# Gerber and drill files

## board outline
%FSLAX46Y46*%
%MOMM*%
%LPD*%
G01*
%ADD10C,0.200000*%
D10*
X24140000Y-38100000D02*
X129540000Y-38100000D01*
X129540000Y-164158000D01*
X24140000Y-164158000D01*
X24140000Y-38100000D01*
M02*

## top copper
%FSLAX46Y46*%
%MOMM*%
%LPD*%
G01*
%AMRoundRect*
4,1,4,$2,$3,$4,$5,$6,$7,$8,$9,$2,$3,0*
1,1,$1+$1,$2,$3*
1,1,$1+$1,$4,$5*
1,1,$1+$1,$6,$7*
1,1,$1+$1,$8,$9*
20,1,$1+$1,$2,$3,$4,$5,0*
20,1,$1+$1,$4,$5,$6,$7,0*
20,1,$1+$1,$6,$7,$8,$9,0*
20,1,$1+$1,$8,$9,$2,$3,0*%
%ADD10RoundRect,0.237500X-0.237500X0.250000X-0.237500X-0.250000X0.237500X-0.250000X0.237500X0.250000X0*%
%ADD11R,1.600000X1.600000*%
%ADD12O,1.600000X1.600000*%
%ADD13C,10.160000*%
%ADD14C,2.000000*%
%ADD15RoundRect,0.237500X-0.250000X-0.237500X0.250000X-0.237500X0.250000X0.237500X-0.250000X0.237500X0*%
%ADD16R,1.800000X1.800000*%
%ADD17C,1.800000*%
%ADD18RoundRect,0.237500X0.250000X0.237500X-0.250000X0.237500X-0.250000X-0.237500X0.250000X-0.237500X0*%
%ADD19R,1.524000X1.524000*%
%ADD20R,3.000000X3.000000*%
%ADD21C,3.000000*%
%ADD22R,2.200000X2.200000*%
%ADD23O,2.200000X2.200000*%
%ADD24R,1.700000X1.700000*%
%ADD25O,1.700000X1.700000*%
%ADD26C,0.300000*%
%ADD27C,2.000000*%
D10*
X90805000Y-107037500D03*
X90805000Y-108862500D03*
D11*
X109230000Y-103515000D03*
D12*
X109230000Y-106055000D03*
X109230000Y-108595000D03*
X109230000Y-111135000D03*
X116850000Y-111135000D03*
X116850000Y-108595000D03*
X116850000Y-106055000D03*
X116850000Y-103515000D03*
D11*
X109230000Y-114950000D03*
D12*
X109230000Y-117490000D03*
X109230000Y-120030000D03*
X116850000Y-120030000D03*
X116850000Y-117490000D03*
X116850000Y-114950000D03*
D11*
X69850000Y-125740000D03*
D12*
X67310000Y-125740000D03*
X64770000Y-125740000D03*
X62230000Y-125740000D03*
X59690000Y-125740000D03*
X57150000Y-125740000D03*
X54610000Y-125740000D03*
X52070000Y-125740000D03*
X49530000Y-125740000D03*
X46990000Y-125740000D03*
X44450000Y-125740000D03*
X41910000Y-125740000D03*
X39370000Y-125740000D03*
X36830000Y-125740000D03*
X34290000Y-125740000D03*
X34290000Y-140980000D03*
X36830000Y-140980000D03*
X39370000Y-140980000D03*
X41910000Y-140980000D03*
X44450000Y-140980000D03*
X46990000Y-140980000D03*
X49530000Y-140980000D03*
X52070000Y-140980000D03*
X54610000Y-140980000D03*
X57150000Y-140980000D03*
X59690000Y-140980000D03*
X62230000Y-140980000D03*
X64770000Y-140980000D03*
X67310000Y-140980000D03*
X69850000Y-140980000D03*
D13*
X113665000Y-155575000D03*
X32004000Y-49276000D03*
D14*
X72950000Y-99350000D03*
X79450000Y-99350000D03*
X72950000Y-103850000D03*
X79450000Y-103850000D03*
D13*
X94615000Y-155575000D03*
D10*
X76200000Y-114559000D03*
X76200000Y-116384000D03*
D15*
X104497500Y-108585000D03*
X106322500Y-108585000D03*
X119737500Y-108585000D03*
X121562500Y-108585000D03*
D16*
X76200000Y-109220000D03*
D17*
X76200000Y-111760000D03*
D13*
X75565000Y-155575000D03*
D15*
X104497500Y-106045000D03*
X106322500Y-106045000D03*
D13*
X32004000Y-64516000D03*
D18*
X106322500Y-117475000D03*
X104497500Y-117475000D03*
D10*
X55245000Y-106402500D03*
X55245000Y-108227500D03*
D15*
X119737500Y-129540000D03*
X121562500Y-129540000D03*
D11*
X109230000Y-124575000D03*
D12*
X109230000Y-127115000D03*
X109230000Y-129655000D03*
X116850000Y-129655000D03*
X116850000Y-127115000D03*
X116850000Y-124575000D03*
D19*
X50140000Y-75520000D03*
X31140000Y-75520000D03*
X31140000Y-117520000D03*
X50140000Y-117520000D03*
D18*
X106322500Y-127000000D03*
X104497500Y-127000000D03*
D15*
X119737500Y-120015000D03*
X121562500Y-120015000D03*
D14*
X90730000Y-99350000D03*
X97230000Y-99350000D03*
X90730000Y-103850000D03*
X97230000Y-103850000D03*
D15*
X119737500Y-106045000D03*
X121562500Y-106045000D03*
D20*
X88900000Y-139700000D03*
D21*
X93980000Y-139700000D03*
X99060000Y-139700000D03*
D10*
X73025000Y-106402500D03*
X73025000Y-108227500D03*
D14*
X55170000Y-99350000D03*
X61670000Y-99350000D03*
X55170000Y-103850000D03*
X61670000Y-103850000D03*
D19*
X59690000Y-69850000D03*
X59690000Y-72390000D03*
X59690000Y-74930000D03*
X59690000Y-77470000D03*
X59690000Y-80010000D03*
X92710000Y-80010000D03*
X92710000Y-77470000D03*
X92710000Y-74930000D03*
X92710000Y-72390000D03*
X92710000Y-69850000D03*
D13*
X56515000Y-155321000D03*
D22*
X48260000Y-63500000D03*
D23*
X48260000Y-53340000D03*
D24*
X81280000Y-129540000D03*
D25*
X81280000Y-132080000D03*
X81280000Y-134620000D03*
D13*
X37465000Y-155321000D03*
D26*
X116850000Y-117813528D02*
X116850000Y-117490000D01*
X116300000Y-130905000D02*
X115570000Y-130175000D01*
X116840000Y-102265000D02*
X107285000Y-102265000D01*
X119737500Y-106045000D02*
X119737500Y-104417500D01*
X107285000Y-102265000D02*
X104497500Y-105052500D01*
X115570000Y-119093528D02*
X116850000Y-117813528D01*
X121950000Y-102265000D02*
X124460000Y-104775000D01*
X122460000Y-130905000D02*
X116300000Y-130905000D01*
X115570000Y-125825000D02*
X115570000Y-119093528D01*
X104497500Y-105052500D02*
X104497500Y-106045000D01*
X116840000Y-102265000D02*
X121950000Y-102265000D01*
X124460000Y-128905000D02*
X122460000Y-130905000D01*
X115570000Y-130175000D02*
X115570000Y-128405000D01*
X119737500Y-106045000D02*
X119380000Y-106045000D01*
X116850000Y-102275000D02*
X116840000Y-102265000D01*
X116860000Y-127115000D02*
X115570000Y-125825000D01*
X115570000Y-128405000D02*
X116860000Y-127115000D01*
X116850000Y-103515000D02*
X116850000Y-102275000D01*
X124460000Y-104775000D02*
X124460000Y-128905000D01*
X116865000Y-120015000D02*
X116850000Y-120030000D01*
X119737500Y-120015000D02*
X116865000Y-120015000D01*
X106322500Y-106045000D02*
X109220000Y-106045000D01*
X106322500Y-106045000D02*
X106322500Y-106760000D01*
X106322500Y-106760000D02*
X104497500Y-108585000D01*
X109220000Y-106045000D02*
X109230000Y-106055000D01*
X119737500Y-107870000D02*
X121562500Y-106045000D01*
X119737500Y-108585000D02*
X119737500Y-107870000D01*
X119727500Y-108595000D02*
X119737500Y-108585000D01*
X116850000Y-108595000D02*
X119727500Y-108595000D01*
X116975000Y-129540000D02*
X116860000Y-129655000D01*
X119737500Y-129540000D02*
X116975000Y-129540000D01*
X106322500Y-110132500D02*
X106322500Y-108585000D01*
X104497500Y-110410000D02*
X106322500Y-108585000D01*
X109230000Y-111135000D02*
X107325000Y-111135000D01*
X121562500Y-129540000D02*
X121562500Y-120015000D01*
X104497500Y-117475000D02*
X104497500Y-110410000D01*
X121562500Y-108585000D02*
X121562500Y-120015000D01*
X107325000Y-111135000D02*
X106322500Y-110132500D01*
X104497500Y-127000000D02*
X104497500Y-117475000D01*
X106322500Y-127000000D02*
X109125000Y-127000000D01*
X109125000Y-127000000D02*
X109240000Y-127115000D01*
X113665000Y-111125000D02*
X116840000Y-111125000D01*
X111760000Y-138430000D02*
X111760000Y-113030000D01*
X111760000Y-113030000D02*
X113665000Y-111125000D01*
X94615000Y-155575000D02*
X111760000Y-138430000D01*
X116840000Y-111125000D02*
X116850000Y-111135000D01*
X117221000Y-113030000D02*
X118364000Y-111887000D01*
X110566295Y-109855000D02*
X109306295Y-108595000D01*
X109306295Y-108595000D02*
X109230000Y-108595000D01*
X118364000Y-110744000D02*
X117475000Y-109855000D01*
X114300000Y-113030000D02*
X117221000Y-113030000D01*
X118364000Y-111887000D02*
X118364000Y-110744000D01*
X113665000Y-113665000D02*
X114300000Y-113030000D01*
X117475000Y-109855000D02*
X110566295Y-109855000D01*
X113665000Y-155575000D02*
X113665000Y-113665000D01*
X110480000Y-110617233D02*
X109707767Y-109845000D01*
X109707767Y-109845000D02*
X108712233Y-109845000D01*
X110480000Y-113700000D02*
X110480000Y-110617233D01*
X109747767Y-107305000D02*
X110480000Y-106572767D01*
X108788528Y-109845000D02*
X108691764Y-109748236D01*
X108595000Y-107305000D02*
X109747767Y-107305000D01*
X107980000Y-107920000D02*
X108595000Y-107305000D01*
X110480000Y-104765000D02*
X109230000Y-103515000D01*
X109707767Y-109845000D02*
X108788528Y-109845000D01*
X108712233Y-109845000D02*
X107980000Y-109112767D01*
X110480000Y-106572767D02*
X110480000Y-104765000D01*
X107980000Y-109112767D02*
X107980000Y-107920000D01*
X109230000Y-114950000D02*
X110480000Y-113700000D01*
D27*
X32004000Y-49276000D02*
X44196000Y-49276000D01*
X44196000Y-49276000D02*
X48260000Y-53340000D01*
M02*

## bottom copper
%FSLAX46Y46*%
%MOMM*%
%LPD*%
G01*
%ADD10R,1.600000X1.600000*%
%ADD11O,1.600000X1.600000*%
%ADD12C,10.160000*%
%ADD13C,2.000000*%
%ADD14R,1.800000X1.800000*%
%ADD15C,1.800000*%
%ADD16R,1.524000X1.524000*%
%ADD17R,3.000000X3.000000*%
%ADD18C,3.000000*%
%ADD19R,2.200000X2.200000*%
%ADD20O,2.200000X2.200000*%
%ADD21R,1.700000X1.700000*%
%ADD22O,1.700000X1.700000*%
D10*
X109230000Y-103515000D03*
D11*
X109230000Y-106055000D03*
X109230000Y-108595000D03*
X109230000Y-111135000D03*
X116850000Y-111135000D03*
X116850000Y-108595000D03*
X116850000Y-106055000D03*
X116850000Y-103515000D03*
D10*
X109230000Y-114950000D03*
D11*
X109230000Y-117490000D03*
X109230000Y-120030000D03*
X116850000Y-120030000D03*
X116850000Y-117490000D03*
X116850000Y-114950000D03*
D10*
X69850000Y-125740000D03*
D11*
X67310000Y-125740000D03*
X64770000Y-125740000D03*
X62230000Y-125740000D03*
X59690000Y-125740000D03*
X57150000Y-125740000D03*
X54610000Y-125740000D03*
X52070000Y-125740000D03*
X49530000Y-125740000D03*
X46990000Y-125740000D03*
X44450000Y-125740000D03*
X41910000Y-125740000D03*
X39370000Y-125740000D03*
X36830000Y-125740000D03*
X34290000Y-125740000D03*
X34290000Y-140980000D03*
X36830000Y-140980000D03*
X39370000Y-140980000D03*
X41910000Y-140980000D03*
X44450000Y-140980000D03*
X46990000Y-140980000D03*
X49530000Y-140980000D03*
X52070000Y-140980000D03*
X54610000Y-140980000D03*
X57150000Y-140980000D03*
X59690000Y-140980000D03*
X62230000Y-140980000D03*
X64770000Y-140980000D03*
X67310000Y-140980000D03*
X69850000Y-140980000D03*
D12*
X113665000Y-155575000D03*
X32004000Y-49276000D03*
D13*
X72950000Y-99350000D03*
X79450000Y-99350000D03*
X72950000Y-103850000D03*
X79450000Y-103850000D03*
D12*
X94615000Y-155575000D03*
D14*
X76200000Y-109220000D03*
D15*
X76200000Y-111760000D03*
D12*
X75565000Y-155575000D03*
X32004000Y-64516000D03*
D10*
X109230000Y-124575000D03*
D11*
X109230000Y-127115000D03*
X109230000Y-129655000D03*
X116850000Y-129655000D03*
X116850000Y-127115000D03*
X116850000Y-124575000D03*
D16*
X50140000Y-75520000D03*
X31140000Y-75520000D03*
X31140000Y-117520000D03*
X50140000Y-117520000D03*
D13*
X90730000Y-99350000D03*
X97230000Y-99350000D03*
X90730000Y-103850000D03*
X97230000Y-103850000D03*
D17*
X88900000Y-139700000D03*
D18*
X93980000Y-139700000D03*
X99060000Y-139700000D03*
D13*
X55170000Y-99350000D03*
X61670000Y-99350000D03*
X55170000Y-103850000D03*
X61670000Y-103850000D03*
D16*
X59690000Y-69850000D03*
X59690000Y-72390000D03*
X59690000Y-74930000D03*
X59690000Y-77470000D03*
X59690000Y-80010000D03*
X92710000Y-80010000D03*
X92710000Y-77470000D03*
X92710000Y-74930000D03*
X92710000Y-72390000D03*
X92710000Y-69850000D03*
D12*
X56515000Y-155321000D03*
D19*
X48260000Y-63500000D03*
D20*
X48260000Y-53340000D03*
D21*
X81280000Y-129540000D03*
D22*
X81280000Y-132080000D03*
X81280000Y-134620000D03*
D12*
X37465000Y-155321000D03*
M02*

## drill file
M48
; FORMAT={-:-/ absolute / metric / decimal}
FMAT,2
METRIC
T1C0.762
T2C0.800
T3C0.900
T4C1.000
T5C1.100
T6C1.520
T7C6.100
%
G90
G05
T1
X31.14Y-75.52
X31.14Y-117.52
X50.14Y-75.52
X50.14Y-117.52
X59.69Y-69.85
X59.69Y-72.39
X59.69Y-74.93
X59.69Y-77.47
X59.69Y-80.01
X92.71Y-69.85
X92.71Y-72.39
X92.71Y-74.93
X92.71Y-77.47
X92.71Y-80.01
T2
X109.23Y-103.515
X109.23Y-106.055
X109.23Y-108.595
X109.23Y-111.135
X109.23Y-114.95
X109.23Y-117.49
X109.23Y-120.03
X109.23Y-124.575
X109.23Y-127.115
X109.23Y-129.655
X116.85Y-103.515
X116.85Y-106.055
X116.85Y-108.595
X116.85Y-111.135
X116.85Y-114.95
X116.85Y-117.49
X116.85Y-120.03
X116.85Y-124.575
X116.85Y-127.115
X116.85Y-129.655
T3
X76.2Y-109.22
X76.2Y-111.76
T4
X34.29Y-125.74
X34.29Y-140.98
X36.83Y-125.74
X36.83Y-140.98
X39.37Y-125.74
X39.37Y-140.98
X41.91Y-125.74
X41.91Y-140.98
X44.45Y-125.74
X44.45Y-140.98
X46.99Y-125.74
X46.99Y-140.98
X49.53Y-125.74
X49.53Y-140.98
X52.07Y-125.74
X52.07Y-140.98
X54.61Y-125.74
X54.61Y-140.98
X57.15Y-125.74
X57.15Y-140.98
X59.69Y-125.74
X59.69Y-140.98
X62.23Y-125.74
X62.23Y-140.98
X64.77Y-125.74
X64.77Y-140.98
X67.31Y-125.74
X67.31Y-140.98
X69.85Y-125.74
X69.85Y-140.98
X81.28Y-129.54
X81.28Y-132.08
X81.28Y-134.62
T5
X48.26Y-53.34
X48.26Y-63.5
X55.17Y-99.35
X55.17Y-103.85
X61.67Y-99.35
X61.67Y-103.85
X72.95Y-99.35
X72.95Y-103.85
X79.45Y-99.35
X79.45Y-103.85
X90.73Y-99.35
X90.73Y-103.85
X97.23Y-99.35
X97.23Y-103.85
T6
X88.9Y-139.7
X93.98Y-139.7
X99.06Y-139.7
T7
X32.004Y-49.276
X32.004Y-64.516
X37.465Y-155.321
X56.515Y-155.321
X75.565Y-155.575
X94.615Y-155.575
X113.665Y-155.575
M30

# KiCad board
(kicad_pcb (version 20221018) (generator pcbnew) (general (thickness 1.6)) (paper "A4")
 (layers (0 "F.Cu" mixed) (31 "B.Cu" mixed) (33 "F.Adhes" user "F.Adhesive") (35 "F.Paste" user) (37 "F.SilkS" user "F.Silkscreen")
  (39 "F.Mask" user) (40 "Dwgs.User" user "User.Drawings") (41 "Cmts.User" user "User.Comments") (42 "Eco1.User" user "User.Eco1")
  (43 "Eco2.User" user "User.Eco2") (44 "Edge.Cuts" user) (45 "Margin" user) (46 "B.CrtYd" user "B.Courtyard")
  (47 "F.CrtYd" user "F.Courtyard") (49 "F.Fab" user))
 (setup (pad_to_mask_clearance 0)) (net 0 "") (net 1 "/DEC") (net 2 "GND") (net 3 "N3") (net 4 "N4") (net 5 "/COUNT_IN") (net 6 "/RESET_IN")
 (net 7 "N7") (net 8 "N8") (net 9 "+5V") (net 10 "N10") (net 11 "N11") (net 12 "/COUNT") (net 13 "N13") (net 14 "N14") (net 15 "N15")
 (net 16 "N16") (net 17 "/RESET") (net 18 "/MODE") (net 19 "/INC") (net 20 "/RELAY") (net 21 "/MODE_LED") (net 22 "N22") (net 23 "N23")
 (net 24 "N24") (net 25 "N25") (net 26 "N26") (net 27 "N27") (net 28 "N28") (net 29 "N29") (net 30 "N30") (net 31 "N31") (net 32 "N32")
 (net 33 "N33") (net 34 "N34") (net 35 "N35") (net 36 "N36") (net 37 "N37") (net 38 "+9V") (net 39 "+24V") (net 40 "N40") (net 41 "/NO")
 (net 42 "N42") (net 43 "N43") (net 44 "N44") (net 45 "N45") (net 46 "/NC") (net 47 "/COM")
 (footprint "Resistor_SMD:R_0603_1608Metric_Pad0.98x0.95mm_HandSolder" (layer "F.Cu") (at 90.805 107.95 -90)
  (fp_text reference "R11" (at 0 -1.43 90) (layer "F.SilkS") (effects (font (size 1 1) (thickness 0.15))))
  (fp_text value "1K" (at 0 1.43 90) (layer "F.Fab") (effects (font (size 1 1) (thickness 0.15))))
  (pad "1" smd roundrect (at -0.9125 0 270) (size 0.975 0.95) (layers "F.Cu" "F.Paste" "F.Mask") (roundrect_rratio 0.25) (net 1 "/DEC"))
  (pad "2" smd roundrect (at 0.9125 0 270) (size 0.975 0.95) (layers "F.Cu" "F.Paste" "F.Mask") (roundrect_rratio 0.25) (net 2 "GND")))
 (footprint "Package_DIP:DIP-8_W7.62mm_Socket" (layer "F.Cu") (at 109.23 103.515)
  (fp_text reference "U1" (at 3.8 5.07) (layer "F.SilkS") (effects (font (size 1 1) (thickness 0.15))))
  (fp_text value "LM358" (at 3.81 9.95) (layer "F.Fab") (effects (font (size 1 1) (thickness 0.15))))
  (pad "1" thru_hole rect (at 0 0) (size 1.6 1.6) (drill 0.8) (layers "*.Cu" "*.Mask") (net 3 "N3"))
  (pad "2" thru_hole oval (at 0 2.54) (size 1.6 1.6) (drill 0.8) (layers "*.Cu" "*.Mask") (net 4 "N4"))
  (pad "3" thru_hole oval (at 0 5.08) (size 1.6 1.6) (drill 0.8) (layers "*.Cu" "*.Mask") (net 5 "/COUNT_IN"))
  (pad "4" thru_hole oval (at 0 7.62) (size 1.6 1.6) (drill 0.8) (layers "*.Cu" "*.Mask") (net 2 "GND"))
  (pad "5" thru_hole oval (at 7.62 7.62) (size 1.6 1.6) (drill 0.8) (layers "*.Cu" "*.Mask") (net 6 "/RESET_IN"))
  (pad "6" thru_hole oval (at 7.62 5.08) (size 1.6 1.6) (drill 0.8) (layers "*.Cu" "*.Mask") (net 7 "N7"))
  (pad "7" thru_hole oval (at 7.62 2.54) (size 1.6 1.6) (drill 0.8) (layers "*.Cu" "*.Mask") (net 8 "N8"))
  (pad "8" thru_hole oval (at 7.62 0) (size 1.6 1.6) (drill 0.8) (layers "*.Cu" "*.Mask") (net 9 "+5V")))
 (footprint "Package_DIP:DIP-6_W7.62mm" (layer "F.Cu") (at 109.23 114.95)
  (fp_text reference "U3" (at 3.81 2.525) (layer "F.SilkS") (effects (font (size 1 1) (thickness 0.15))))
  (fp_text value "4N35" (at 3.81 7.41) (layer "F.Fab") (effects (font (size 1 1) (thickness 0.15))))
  (pad "1" thru_hole rect (at 0 0) (size 1.6 1.6) (drill 0.8) (layers "*.Cu" "*.Mask") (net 3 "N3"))
  (pad "2" thru_hole oval (at 0 2.54) (size 1.6 1.6) (drill 0.8) (layers "*.Cu" "*.Mask") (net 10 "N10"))
  (pad "3" thru_hole oval (at 0 5.08) (size 1.6 1.6) (drill 0.8) (layers "*.Cu" "*.Mask") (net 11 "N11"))
  (pad "4" thru_hole oval (at 7.62 5.08) (size 1.6 1.6) (drill 0.8) (layers "*.Cu" "*.Mask") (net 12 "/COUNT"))
  (pad "5" thru_hole oval (at 7.62 2.54) (size 1.6 1.6) (drill 0.8) (layers "*.Cu" "*.Mask") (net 9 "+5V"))
  (pad "6" thru_hole oval (at 7.62 0) (size 1.6 1.6) (drill 0.8) (layers "*.Cu" "*.Mask") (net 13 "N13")))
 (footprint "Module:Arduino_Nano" (layer "F.Cu") (at 69.85 125.74 -90)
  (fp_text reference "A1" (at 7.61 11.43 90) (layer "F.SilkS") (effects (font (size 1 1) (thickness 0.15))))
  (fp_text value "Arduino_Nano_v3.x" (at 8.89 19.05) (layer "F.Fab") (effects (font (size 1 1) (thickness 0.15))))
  (pad "1" thru_hole rect (at 0 0 270) (size 1.6 1.6) (drill 1) (layers "*.Cu" "*.Mask") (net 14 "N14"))
  (pad "2" thru_hole oval (at 0 2.54 270) (size 1.6 1.6) (drill 1) (layers "*.Cu" "*.Mask") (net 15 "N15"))
  (pad "3" thru_hole oval (at 0 5.08 270) (size 1.6 1.6) (drill 1) (layers "*.Cu" "*.Mask") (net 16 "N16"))
  (pad "4" thru_hole oval (at 0 7.62 270) (size 1.6 1.6) (drill 1) (layers "*.Cu" "*.Mask") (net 2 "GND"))
  (pad "5" thru_hole oval (at 0 10.16 270) (size 1.6 1.6) (drill 1) (layers "*.Cu" "*.Mask") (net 12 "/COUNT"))
  (pad "6" thru_hole oval (at 0 12.7 270) (size 1.6 1.6) (drill 1) (layers "*.Cu" "*.Mask") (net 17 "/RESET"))
  (pad "7" thru_hole oval (at 0 15.24 270) (size 1.6 1.6) (drill 1) (layers "*.Cu" "*.Mask") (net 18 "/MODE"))
  (pad "8" thru_hole oval (at 0 17.78 270) (size 1.6 1.6) (drill 1) (layers "*.Cu" "*.Mask") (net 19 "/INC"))
  (pad "9" thru_hole oval (at 0 20.32 270) (size 1.6 1.6) (drill 1) (layers "*.Cu" "*.Mask") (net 1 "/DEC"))
  (pad "10" thru_hole oval (at 0 22.86 270) (size 1.6 1.6) (drill 1) (layers "*.Cu" "*.Mask") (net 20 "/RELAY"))
  (pad "11" thru_hole oval (at 0 25.4 270) (size 1.6 1.6) (drill 1) (layers "*.Cu" "*.Mask") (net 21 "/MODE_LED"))
  (pad "12" thru_hole oval (at 0 27.94 270) (size 1.6 1.6) (drill 1) (layers "*.Cu" "*.Mask") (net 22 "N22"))
  (pad "13" thru_hole oval (at 0 30.48 270) (size 1.6 1.6) (drill 1) (layers "*.Cu" "*.Mask") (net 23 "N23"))
  (pad "14" thru_hole oval (at 0 33.02 270) (size 1.6 1.6) (drill 1) (layers "*.Cu" "*.Mask") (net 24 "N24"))
  (pad "15" thru_hole oval (at 0 35.56 270) (size 1.6 1.6) (drill 1) (layers "*.Cu" "*.Mask") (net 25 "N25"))
  (pad "16" thru_hole oval (at 15.24 35.56 270) (size 1.6 1.6) (drill 1) (layers "*.Cu" "*.Mask") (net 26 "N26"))
  (pad "17" thru_hole oval (at 15.24 33.02 270) (size 1.6 1.6) (drill 1) (layers "*.Cu" "*.Mask") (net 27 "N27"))
  (pad "18" thru_hole oval (at 15.24 30.48 270) (size 1.6 1.6) (drill 1) (layers "*.Cu" "*.Mask") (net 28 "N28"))
  (pad "19" thru_hole oval (at 15.24 27.94 270) (size 1.6 1.6) (drill 1) (layers "*.Cu" "*.Mask") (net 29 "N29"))
  (pad "20" thru_hole oval (at 15.24 25.4 270) (size 1.6 1.6) (drill 1) (layers "*.Cu" "*.Mask") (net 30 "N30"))
  (pad "21" thru_hole oval (at 15.24 22.86 270) (size 1.6 1.6) (drill 1) (layers "*.Cu" "*.Mask") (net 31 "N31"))
  (pad "22" thru_hole oval (at 15.24 20.32 270) (size 1.6 1.6) (drill 1) (layers "*.Cu" "*.Mask") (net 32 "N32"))
  (pad "23" thru_hole oval (at 15.24 17.78 270) (size 1.6 1.6) (drill 1) (layers "*.Cu" "*.Mask") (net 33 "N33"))
  (pad "24" thru_hole oval (at 15.24 15.24 270) (size 1.6 1.6) (drill 1) (layers "*.Cu" "*.Mask") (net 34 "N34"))
  (pad "25" thru_hole oval (at 15.24 12.7 270) (size 1.6 1.6) (drill 1) (layers "*.Cu" "*.Mask") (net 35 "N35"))
  (pad "26" thru_hole oval (at 15.24 10.16 270) (size 1.6 1.6) (drill 1) (layers "*.Cu" "*.Mask") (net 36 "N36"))
  (pad "27" thru_hole oval (at 15.24 7.62 270) (size 1.6 1.6) (drill 1) (layers "*.Cu" "*.Mask") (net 9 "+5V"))
  (pad "28" thru_hole oval (at 15.24 5.08 270) (size 1.6 1.6) (drill 1) (layers "*.Cu" "*.Mask") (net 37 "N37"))
  (pad "29" thru_hole oval (at 15.24 2.54 270) (size 1.6 1.6) (drill 1) (layers "*.Cu" "*.Mask") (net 2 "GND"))
  (pad "30" thru_hole oval (at 15.24 0 270) (size 1.6 1.6) (drill 1) (layers "*.Cu" "*.Mask") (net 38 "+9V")))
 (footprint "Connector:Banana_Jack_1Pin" (layer "F.Cu") (at 113.665 155.575)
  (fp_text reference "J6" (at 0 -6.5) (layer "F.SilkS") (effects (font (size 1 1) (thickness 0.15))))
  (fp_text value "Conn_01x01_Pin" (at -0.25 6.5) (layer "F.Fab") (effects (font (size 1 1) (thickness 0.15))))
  (pad "1" thru_hole circle (at 0 0) (size 10.16 10.16) (drill 6.1) (layers "*.Cu" "*.Mask") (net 5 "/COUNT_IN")))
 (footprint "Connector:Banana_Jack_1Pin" (layer "F.Cu") (at 32.004 49.276)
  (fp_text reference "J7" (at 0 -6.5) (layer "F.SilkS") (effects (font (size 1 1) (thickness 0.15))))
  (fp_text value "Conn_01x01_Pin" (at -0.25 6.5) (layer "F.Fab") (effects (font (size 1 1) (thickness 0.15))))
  (pad "1" thru_hole circle (at 0 0) (size 10.16 10.16) (drill 6.1) (layers "*.Cu" "*.Mask") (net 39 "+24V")))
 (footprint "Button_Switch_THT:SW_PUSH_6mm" (layer "F.Cu") (at 72.95 99.35)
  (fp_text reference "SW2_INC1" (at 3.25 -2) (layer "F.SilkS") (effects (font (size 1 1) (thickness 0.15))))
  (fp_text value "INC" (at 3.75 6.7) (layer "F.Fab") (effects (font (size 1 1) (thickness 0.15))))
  (pad "1" thru_hole circle (at 0 0 90) (size 2 2) (drill 1.1) (layers "*.Cu" "*.Mask") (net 9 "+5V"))
  (pad "1" thru_hole circle (at 6.5 0 90) (size 2 2) (drill 1.1) (layers "*.Cu" "*.Mask") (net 9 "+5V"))
  (pad "2" thru_hole circle (at 0 4.5 90) (size 2 2) (drill 1.1) (layers "*.Cu" "*.Mask") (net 19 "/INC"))
  (pad "2" thru_hole circle (at 6.5 4.5 90) (size 2 2) (drill 1.1) (layers "*.Cu" "*.Mask") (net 19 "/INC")))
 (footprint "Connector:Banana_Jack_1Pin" (layer "F.Cu") (at 94.615 155.575)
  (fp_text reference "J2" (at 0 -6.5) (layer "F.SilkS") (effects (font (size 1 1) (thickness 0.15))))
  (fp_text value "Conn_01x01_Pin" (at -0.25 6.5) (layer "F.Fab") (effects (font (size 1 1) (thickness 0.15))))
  (pad "1" thru_hole circle (at 0 0) (size 10.16 10.16) (drill 6.1) (layers "*.Cu" "*.Mask") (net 6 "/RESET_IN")))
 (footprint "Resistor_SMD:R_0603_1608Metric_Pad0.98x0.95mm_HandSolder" (layer "F.Cu") (at 76.2 115.4715 -90)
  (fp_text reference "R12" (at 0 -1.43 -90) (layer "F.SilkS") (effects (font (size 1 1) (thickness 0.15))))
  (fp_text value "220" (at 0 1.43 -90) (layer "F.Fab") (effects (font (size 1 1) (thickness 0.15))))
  (pad "1" smd roundrect (at -0.9125 0 270) (size 0.975 0.95) (layers "F.Cu" "F.Paste" "F.Mask") (roundrect_rratio 0.25) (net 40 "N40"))
  (pad "2" smd roundrect (at 0.9125 0 270) (size 0.975 0.95) (layers "F.Cu" "F.Paste" "F.Mask") (roundrect_rratio 0.25) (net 2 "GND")))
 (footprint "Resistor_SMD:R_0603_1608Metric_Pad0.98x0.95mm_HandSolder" (layer "F.Cu") (at 105.41 108.585)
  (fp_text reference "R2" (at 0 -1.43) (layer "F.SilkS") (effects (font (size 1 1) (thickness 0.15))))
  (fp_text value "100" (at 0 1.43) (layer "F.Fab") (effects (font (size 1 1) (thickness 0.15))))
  (pad "1" smd roundrect (at -0.9125 0) (size 0.975 0.95) (layers "F.Cu" "F.Paste" "F.Mask") (roundrect_rratio 0.25) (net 4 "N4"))
  (pad "2" smd roundrect (at 0.9125 0) (size 0.975 0.95) (layers "F.Cu" "F.Paste" "F.Mask") (roundrect_rratio 0.25) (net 2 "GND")))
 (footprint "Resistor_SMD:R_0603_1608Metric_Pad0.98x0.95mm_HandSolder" (layer "F.Cu") (at 120.65 108.585)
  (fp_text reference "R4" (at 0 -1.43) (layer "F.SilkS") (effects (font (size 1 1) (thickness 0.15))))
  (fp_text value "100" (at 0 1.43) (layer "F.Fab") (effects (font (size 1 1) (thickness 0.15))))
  (pad "1" smd roundrect (at -0.9125 0) (size 0.975 0.95) (layers "F.Cu" "F.Paste" "F.Mask") (roundrect_rratio 0.25) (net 7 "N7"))
  (pad "2" smd roundrect (at 0.9125 0) (size 0.975 0.95) (layers "F.Cu" "F.Paste" "F.Mask") (roundrect_rratio 0.25) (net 2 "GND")))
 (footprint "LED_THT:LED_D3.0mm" (layer "F.Cu") (at 76.2 109.22 -90)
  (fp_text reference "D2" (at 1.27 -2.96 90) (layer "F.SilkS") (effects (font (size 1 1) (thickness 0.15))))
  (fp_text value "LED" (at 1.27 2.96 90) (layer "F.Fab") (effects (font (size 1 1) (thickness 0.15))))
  (pad "1" thru_hole rect (at 0 0 270) (size 1.8 1.8) (drill 0.9) (layers "*.Cu" "*.Mask") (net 21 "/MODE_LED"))
  (pad "2" thru_hole circle (at 2.54 0 270) (size 1.8 1.8) (drill 0.9) (layers "*.Cu" "*.Mask") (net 40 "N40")))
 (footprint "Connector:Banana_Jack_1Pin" (layer "F.Cu") (at 75.565 155.575)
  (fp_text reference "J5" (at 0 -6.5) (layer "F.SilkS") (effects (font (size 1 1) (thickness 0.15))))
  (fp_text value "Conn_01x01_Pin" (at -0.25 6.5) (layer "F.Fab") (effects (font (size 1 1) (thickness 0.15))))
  (pad "1" thru_hole circle (at 0 0) (size 10.16 10.16) (drill 6.1) (layers "*.Cu" "*.Mask") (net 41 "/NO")))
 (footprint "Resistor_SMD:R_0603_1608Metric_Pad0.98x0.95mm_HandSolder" (layer "F.Cu") (at 105.41 106.045)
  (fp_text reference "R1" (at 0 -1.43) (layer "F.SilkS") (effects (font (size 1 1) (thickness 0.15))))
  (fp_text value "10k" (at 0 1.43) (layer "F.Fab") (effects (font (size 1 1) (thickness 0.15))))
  (pad "1" smd roundrect (at -0.9125 0) (size 0.975 0.95) (layers "F.Cu" "F.Paste" "F.Mask") (roundrect_rratio 0.25) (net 9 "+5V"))
  (pad "2" smd roundrect (at 0.9125 0) (size 0.975 0.95) (layers "F.Cu" "F.Paste" "F.Mask") (roundrect_rratio 0.25) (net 4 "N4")))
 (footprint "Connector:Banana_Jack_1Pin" (layer "F.Cu") (at 32.004 64.516)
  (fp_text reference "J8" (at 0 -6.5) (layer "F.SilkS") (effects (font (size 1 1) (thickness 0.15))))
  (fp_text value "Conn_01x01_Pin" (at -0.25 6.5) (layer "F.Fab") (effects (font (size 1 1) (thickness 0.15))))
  (pad "1" thru_hole circle (at 0 0) (size 10.16 10.16) (drill 6.1) (layers "*.Cu" "*.Mask") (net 2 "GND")))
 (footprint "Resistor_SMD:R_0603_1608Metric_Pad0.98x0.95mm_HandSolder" (layer "F.Cu") (at 105.41 117.475 180)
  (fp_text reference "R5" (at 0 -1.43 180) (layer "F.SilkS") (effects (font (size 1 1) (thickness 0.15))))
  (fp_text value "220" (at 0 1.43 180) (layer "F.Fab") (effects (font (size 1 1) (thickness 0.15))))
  (pad "1" smd roundrect (at -0.9125 0 180) (size 0.975 0.95) (layers "F.Cu" "F.Paste" "F.Mask") (roundrect_rratio 0.25) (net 10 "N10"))
  (pad "2" smd roundrect (at 0.9125 0 180) (size 0.975 0.95) (layers "F.Cu" "F.Paste" "F.Mask") (roundrect_rratio 0.25) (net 2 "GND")))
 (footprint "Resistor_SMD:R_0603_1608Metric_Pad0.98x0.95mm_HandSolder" (layer "F.Cu") (at 55.245 107.315 -90)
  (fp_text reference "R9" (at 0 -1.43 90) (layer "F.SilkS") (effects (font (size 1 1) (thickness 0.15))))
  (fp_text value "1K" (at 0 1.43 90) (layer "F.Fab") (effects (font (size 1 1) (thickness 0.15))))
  (pad "1" smd roundrect (at -0.9125 0 270) (size 0.975 0.95) (layers "F.Cu" "F.Paste" "F.Mask") (roundrect_rratio 0.25) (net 18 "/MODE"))
  (pad "2" smd roundrect (at 0.9125 0 270) (size 0.975 0.95) (layers "F.Cu" "F.Paste" "F.Mask") (roundrect_rratio 0.25) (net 2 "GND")))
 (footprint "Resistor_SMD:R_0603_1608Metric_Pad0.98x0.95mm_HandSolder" (layer "F.Cu") (at 120.65 129.54)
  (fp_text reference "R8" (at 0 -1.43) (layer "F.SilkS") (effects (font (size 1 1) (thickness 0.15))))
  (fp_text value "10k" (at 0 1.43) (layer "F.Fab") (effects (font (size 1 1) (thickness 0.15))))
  (pad "1" smd roundrect (at -0.9125 0) (size 0.975 0.95) (layers "F.Cu" "F.Paste" "F.Mask") (roundrect_rratio 0.25) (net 17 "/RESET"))
  (pad "2" smd roundrect (at 0.9125 0) (size 0.975 0.95) (layers "F.Cu" "F.Paste" "F.Mask") (roundrect_rratio 0.25) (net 2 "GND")))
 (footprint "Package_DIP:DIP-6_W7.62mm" (layer "F.Cu") (at 109.23 124.575)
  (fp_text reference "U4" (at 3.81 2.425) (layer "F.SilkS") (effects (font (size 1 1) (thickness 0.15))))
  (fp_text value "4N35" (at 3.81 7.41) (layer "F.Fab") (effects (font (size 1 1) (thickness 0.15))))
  (pad "1" thru_hole rect (at 0 0) (size 1.6 1.6) (drill 0.8) (layers "*.Cu" "*.Mask") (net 8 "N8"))
  (pad "2" thru_hole oval (at 0 2.54) (size 1.6 1.6) (drill 0.8) (layers "*.Cu" "*.Mask") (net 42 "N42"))
  (pad "3" thru_hole oval (at 0 5.08) (size 1.6 1.6) (drill 0.8) (layers "*.Cu" "*.Mask") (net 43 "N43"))
  (pad "4" thru_hole oval (at 7.62 5.08) (size 1.6 1.6) (drill 0.8) (layers "*.Cu" "*.Mask") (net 17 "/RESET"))
  (pad "5" thru_hole oval (at 7.62 2.54) (size 1.6 1.6) (drill 0.8) (layers "*.Cu" "*.Mask") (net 9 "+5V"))
  (pad "6" thru_hole oval (at 7.62 0) (size 1.6 1.6) (drill 0.8) (layers "*.Cu" "*.Mask") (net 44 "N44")))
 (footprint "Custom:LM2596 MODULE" (layer "F.Cu") (at 40.64 96.52 -90)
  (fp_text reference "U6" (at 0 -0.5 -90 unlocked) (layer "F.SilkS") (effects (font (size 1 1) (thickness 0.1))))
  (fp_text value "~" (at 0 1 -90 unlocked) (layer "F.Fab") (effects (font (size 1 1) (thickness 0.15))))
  (pad "1" thru_hole rect (at -21 -9.5 270) (size 1.524 1.524) (drill 0.762) (layers "*.Cu" "*.Mask") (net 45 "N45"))
  (pad "2" thru_hole rect (at -21 9.5 270) (size 1.524 1.524) (drill 0.762) (layers "*.Cu" "*.Mask") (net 2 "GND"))
  (pad "3" thru_hole rect (at 21 9.5 270) (size 1.524 1.524) (drill 0.762) (layers "*.Cu" "*.Mask") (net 2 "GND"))
  (pad "4" thru_hole rect (at 21 -9.5 270) (size 1.524 1.524) (drill 0.762) (layers "*.Cu" "*.Mask") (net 38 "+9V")))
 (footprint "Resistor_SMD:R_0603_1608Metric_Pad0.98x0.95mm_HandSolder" (layer "F.Cu") (at 105.41 127 180)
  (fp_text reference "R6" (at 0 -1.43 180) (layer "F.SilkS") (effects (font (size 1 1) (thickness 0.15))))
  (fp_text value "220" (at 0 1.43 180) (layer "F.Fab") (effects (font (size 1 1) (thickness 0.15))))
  (pad "1" smd roundrect (at -0.9125 0 180) (size 0.975 0.95) (layers "F.Cu" "F.Paste" "F.Mask") (roundrect_rratio 0.25) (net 42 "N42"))
  (pad "2" smd roundrect (at 0.9125 0 180) (size 0.975 0.95) (layers "F.Cu" "F.Paste" "F.Mask") (roundrect_rratio 0.25) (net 2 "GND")))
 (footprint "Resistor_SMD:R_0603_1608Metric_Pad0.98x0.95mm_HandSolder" (layer "F.Cu") (at 120.65 120.015)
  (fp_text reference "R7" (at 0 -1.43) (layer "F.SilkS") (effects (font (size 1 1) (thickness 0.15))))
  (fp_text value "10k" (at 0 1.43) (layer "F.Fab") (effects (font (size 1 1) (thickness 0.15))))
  (pad "1" smd roundrect (at -0.9125 0) (size 0.975 0.95) (layers "F.Cu" "F.Paste" "F.Mask") (roundrect_rratio 0.25) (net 12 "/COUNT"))
  (pad "2" smd roundrect (at 0.9125 0) (size 0.975 0.95) (layers "F.Cu" "F.Paste" "F.Mask") (roundrect_rratio 0.25) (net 2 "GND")))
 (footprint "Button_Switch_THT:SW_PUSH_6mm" (layer "F.Cu") (at 90.73 99.35)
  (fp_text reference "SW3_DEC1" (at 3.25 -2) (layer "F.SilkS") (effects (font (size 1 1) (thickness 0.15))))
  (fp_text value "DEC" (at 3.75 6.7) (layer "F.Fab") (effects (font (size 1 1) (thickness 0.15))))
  (pad "1" thru_hole circle (at 0 0 90) (size 2 2) (drill 1.1) (layers "*.Cu" "*.Mask") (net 9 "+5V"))
  (pad "1" thru_hole circle (at 6.5 0 90) (size 2 2) (drill 1.1) (layers "*.Cu" "*.Mask") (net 9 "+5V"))
  (pad "2" thru_hole circle (at 0 4.5 90) (size 2 2) (drill 1.1) (layers "*.Cu" "*.Mask") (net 1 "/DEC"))
  (pad "2" thru_hole circle (at 6.5 4.5 90) (size 2 2) (drill 1.1) (layers "*.Cu" "*.Mask") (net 1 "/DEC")))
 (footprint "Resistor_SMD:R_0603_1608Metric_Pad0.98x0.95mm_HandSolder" (layer "F.Cu") (at 120.65 106.045)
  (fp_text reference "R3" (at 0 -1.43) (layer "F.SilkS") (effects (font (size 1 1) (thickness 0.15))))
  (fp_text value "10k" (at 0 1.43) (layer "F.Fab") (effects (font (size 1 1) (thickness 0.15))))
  (pad "1" smd roundrect (at -0.9125 0) (size 0.975 0.95) (layers "F.Cu" "F.Paste" "F.Mask") (roundrect_rratio 0.25) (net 9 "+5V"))
  (pad "2" smd roundrect (at 0.9125 0) (size 0.975 0.95) (layers "F.Cu" "F.Paste" "F.Mask") (roundrect_rratio 0.25) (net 7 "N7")))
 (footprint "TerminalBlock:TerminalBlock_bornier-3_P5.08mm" (layer "F.Cu") (at 88.9 139.7)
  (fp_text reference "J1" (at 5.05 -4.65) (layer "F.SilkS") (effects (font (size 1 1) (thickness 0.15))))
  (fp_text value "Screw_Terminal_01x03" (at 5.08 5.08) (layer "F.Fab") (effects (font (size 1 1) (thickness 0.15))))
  (pad "1" thru_hole rect (at 0 0) (size 3 3) (drill 1.52) (layers "*.Cu" "*.Mask") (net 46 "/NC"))
  (pad "2" thru_hole circle (at 5.08 0) (size 3 3) (drill 1.52) (layers "*.Cu" "*.Mask") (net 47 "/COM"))
  (pad "3" thru_hole circle (at 10.16 0) (size 3 3) (drill 1.52) (layers "*.Cu" "*.Mask") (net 41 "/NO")))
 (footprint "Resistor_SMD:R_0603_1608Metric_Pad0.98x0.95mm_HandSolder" (layer "F.Cu") (at 73.025 107.315 -90)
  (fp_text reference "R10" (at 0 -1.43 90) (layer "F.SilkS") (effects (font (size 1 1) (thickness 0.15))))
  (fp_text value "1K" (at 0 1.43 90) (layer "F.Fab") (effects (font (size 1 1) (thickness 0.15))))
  (pad "1" smd roundrect (at -0.9125 0 270) (size 0.975 0.95) (layers "F.Cu" "F.Paste" "F.Mask") (roundrect_rratio 0.25) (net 19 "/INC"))
  (pad "2" smd roundrect (at 0.9125 0 270) (size 0.975 0.95) (layers "F.Cu" "F.Paste" "F.Mask") (roundrect_rratio 0.25) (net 2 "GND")))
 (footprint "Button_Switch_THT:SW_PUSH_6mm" (layer "F.Cu") (at 55.17 99.35)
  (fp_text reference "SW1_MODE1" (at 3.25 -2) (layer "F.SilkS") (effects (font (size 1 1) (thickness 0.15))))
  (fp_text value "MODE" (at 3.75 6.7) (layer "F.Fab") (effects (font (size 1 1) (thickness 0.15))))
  (pad "1" thru_hole circle (at 0 0 90) (size 2 2) (drill 1.1) (layers "*.Cu" "*.Mask") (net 9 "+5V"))
  (pad "1" thru_hole circle (at 6.5 0 90) (size 2 2) (drill 1.1) (layers "*.Cu" "*.Mask") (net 9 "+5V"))
  (pad "2" thru_hole circle (at 0 4.5 90) (size 2 2) (drill 1.1) (layers "*.Cu" "*.Mask") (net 18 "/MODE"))
  (pad "2" thru_hole circle (at 6.5 4.5 90) (size 2 2) (drill 1.1) (layers "*.Cu" "*.Mask") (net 18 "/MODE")))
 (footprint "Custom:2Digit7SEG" (layer "F.Cu") (at 76.2 69.85)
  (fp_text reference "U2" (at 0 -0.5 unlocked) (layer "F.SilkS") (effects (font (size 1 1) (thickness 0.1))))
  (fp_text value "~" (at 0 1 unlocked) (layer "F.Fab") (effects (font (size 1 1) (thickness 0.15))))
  (pad "1" thru_hole rect (at -16.51 0) (size 1.524 1.524) (drill 0.762) (layers "*.Cu" "*.Mask") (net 9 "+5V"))
  (pad "2" thru_hole rect (at -16.51 2.54) (size 1.524 1.524) (drill 0.762) (layers "*.Cu" "*.Mask") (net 2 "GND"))
  (pad "3" thru_hole rect (at -16.51 5.08) (size 1.524 1.524) (drill 0.762) (layers "*.Cu" "*.Mask") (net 22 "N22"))
  (pad "4" thru_hole rect (at -16.51 7.62) (size 1.524 1.524) (drill 0.762) (layers "*.Cu" "*.Mask") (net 23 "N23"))
  (pad "5" thru_hole rect (at -16.51 10.16) (size 1.524 1.524) (drill 0.762) (layers "*.Cu" "*.Mask") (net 24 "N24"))
  (pad "6" thru_hole rect (at 16.51 10.16) (size 1.524 1.524) (drill 0.762) (layers "*.Cu" "*.Mask"))
  (pad "7" thru_hole rect (at 16.51 7.62) (size 1.524 1.524) (drill 0.762) (layers "*.Cu" "*.Mask"))
  (pad "8" thru_hole rect (at 16.51 5.08) (size 1.524 1.524) (drill 0.762) (layers "*.Cu" "*.Mask"))
  (pad "9" thru_hole rect (at 16.51 2.54) (size 1.524 1.524) (drill 0.762) (layers "*.Cu" "*.Mask"))
  (pad "10" thru_hole rect (at 16.51 0) (size 1.524 1.524) (drill 0.762) (layers "*.Cu" "*.Mask")))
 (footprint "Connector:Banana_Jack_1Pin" (layer "F.Cu") (at 56.515 155.321)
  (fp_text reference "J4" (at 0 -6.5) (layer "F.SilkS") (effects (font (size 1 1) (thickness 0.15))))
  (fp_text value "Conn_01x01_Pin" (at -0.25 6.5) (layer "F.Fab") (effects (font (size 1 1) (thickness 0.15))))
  (pad "1" thru_hole circle (at 0 0) (size 10.16 10.16) (drill 6.1) (layers "*.Cu" "*.Mask") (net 47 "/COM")))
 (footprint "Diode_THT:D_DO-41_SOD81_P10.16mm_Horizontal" (layer "F.Cu") (at 48.26 63.5 90)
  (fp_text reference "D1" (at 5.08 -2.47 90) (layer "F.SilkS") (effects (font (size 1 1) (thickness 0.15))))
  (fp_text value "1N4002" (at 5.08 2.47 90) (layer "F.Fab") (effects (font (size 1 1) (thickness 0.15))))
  (pad "1" thru_hole rect (at 0 0 90) (size 2.2 2.2) (drill 1.1) (layers "*.Cu" "*.Mask") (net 45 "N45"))
  (pad "2" thru_hole oval (at 10.16 0 90) (size 2.2 2.2) (drill 1.1) (layers "*.Cu" "*.Mask") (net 39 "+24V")))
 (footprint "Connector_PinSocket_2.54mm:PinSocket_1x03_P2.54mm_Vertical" (layer "F.Cu") (at 81.28 129.54)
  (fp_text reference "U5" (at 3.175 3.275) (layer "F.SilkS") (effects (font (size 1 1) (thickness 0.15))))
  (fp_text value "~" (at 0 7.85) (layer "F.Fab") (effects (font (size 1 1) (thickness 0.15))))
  (pad "1" thru_hole rect (at 0 0) (size 1.7 1.7) (drill 1) (layers "*.Cu" "*.Mask") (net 20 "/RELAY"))
  (pad "2" thru_hole oval (at 0 2.54) (size 1.7 1.7) (drill 1) (layers "*.Cu" "*.Mask") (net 2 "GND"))
  (pad "3" thru_hole oval (at 0 5.08) (size 1.7 1.7) (drill 1) (layers "*.Cu" "*.Mask") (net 9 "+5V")))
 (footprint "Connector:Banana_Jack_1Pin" (layer "F.Cu") (at 37.465 155.321)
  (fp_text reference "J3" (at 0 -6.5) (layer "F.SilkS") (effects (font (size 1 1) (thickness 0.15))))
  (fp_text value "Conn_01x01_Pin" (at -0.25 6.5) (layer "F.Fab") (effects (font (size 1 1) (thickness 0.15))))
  (pad "1" thru_hole circle (at 0 0) (size 10.16 10.16) (drill 6.1) (layers "*.Cu" "*.Mask") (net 46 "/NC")))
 (gr_rect (start 24.14 38.1) (end 129.54 164.158) (stroke (width 0.2) (type default)) (fill none) (layer "Edge.Cuts"))
 (segment (start 116.85 117.813528) (end 116.85 117.49) (width 0.3) (layer "F.Cu") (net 9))
 (segment (start 116.3 130.905) (end 115.57 130.175) (width 0.3) (layer "F.Cu") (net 9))
 (segment (start 116.84 102.265) (end 107.285 102.265) (width 0.3) (layer "F.Cu") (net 9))
 (segment (start 119.7375 106.045) (end 119.7375 104.4175) (width 0.3) (layer "F.Cu") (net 9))
 (segment (start 107.285 102.265) (end 104.4975 105.0525) (width 0.3) (layer "F.Cu") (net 9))
 (segment (start 115.57 119.093528) (end 116.85 117.813528) (width 0.3) (layer "F.Cu") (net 9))
 (segment (start 121.95 102.265) (end 124.46 104.775) (width 0.3) (layer "F.Cu") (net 9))
 (segment (start 122.46 130.905) (end 116.3 130.905) (width 0.3) (layer "F.Cu") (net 9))
 (segment (start 115.57 125.825) (end 115.57 119.093528) (width 0.3) (layer "F.Cu") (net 9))
 (segment (start 104.4975 105.0525) (end 104.4975 106.045) (width 0.3) (layer "F.Cu") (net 9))
 (segment (start 116.84 102.265) (end 121.95 102.265) (width 0.3) (layer "F.Cu") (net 9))
 (segment (start 124.46 128.905) (end 122.46 130.905) (width 0.3) (layer "F.Cu") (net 9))
 (segment (start 115.57 130.175) (end 115.57 128.405) (width 0.3) (layer "F.Cu") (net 9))
 (segment (start 119.7375 106.045) (end 119.38 106.045) (width 0.3) (layer "F.Cu") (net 9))
 (segment (start 116.85 102.275) (end 116.84 102.265) (width 0.3) (layer "F.Cu") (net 9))
 (segment (start 116.86 127.115) (end 115.57 125.825) (width 0.3) (layer "F.Cu") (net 9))
 (segment (start 115.57 128.405) (end 116.86 127.115) (width 0.3) (layer "F.Cu") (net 9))
 (segment (start 116.85 103.515) (end 116.85 102.275) (width 0.3) (layer "F.Cu") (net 9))
 (segment (start 124.46 104.775) (end 124.46 128.905) (width 0.3) (layer "F.Cu") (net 9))
 (segment (start 116.865 120.015) (end 116.85 120.03) (width 0.3) (layer "F.Cu") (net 12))
 (segment (start 119.7375 120.015) (end 116.865 120.015) (width 0.3) (layer "F.Cu") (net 12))
 (segment (start 106.3225 106.045) (end 109.22 106.045) (width 0.3) (layer "F.Cu") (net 4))
 (segment (start 106.3225 106.045) (end 106.3225 106.76) (width 0.3) (layer "F.Cu") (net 4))
 (segment (start 106.3225 106.76) (end 104.4975 108.585) (width 0.3) (layer "F.Cu") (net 4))
 (segment (start 109.22 106.045) (end 109.23 106.055) (width 0.3) (layer "F.Cu") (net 4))
 (segment (start 119.7375 107.87) (end 121.5625 106.045) (width 0.3) (layer "F.Cu") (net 7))
 (segment (start 119.7375 108.585) (end 119.7375 107.87) (width 0.3) (layer "F.Cu") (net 7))
 (segment (start 119.7275 108.595) (end 119.7375 108.585) (width 0.3) (layer "F.Cu") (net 7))
 (segment (start 116.85 108.595) (end 119.7275 108.595) (width 0.3) (layer "F.Cu") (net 7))
 (segment (start 116.975 129.54) (end 116.86 129.655) (width 0.3) (layer "F.Cu") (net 17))
 (segment (start 119.7375 129.54) (end 116.975 129.54) (width 0.3) (layer "F.Cu") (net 17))
 (segment (start 106.3225 110.1325) (end 106.3225 108.585) (width 0.3) (layer "F.Cu") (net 2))
 (segment (start 104.4975 110.41) (end 106.3225 108.585) (width 0.3) (layer "F.Cu") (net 2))
 (segment (start 109.23 111.135) (end 107.325 111.135) (width 0.3) (layer "F.Cu") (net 2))
 (segment (start 121.5625 129.54) (end 121.5625 120.015) (width 0.3) (layer "F.Cu") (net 2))
 (segment (start 104.4975 117.475) (end 104.4975 110.41) (width 0.3) (layer "F.Cu") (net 2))
 (segment (start 121.5625 108.585) (end 121.5625 120.015) (width 0.3) (layer "F.Cu") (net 2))
 (segment (start 107.325 111.135) (end 106.3225 110.1325) (width 0.3) (layer "F.Cu") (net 2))
 (segment (start 104.4975 127) (end 104.4975 117.475) (width 0.3) (layer "F.Cu") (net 2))
 (segment (start 106.3225 127) (end 109.125 127) (width 0.3) (layer "F.Cu") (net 42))
 (segment (start 109.125 127) (end 109.24 127.115) (width 0.3) (layer "F.Cu") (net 42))
 (segment (start 113.665 111.125) (end 116.84 111.125) (width 0.3) (layer "F.Cu") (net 6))
 (segment (start 111.76 138.43) (end 111.76 113.03) (width 0.3) (layer "F.Cu") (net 6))
 (segment (start 111.76 113.03) (end 113.665 111.125) (width 0.3) (layer "F.Cu") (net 6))
 (segment (start 94.615 155.575) (end 111.76 138.43) (width 0.3) (layer "F.Cu") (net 6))
 (segment (start 116.84 111.125) (end 116.85 111.135) (width 0.3) (layer "F.Cu") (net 6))
 (segment (start 117.221 113.03) (end 118.364 111.887) (width 0.3) (layer "F.Cu") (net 5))
 (segment (start 110.566295 109.855) (end 109.306295 108.595) (width 0.3) (layer "F.Cu") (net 5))
 (segment (start 109.306295 108.595) (end 109.23 108.595) (width 0.3) (layer "F.Cu") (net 5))
 (segment (start 118.364 110.744) (end 117.475 109.855) (width 0.3) (layer "F.Cu") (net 5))
 (segment (start 114.3 113.03) (end 117.221 113.03) (width 0.3) (layer "F.Cu") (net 5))
 (segment (start 118.364 111.887) (end 118.364 110.744) (width 0.3) (layer "F.Cu") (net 5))
 (segment (start 113.665 113.665) (end 114.3 113.03) (width 0.3) (layer "F.Cu") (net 5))
 (segment (start 117.475 109.855) (end 110.566295 109.855) (width 0.3) (layer "F.Cu") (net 5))
 (segment (start 113.665 155.575) (end 113.665 113.665) (width 0.3) (layer "F.Cu") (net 5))
 (segment (start 110.48 110.617233) (end 109.707767 109.845) (width 0.3) (layer "F.Cu") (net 3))
 (segment (start 109.707767 109.845) (end 108.712233 109.845) (width 0.3) (layer "F.Cu") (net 3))
 (segment (start 110.48 113.7) (end 110.48 110.617233) (width 0.3) (layer "F.Cu") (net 3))
 (segment (start 109.747767 107.305) (end 110.48 106.572767) (width 0.3) (layer "F.Cu") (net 3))
 (segment (start 108.788528 109.845) (end 108.691764 109.748236) (width 0.3) (layer "F.Cu") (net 3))
 (segment (start 108.595 107.305) (end 109.747767 107.305) (width 0.3) (layer "F.Cu") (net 3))
 (segment (start 107.98 107.92) (end 108.595 107.305) (width 0.3) (layer "F.Cu") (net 3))
 (segment (start 110.48 104.765) (end 109.23 103.515) (width 0.3) (layer "F.Cu") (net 3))
 (segment (start 109.707767 109.845) (end 108.788528 109.845) (width 0.3) (layer "F.Cu") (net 3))
 (segment (start 108.712233 109.845) (end 107.98 109.112767) (width 0.3) (layer "F.Cu") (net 3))
 (segment (start 110.48 106.572767) (end 110.48 104.765) (width 0.3) (layer "F.Cu") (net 3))
 (segment (start 107.98 109.112767) (end 107.98 107.92) (width 0.3) (layer "F.Cu") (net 3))
 (segment (start 109.23 114.95) (end 110.48 113.7) (width 0.3) (layer "F.Cu") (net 3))
 (segment (start 32.004 49.276) (end 44.196 49.276) (width 2) (layer "F.Cu") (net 39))
 (segment (start 44.196 49.276) (end 48.26 53.34) (width 2) (layer "F.Cu") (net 39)))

